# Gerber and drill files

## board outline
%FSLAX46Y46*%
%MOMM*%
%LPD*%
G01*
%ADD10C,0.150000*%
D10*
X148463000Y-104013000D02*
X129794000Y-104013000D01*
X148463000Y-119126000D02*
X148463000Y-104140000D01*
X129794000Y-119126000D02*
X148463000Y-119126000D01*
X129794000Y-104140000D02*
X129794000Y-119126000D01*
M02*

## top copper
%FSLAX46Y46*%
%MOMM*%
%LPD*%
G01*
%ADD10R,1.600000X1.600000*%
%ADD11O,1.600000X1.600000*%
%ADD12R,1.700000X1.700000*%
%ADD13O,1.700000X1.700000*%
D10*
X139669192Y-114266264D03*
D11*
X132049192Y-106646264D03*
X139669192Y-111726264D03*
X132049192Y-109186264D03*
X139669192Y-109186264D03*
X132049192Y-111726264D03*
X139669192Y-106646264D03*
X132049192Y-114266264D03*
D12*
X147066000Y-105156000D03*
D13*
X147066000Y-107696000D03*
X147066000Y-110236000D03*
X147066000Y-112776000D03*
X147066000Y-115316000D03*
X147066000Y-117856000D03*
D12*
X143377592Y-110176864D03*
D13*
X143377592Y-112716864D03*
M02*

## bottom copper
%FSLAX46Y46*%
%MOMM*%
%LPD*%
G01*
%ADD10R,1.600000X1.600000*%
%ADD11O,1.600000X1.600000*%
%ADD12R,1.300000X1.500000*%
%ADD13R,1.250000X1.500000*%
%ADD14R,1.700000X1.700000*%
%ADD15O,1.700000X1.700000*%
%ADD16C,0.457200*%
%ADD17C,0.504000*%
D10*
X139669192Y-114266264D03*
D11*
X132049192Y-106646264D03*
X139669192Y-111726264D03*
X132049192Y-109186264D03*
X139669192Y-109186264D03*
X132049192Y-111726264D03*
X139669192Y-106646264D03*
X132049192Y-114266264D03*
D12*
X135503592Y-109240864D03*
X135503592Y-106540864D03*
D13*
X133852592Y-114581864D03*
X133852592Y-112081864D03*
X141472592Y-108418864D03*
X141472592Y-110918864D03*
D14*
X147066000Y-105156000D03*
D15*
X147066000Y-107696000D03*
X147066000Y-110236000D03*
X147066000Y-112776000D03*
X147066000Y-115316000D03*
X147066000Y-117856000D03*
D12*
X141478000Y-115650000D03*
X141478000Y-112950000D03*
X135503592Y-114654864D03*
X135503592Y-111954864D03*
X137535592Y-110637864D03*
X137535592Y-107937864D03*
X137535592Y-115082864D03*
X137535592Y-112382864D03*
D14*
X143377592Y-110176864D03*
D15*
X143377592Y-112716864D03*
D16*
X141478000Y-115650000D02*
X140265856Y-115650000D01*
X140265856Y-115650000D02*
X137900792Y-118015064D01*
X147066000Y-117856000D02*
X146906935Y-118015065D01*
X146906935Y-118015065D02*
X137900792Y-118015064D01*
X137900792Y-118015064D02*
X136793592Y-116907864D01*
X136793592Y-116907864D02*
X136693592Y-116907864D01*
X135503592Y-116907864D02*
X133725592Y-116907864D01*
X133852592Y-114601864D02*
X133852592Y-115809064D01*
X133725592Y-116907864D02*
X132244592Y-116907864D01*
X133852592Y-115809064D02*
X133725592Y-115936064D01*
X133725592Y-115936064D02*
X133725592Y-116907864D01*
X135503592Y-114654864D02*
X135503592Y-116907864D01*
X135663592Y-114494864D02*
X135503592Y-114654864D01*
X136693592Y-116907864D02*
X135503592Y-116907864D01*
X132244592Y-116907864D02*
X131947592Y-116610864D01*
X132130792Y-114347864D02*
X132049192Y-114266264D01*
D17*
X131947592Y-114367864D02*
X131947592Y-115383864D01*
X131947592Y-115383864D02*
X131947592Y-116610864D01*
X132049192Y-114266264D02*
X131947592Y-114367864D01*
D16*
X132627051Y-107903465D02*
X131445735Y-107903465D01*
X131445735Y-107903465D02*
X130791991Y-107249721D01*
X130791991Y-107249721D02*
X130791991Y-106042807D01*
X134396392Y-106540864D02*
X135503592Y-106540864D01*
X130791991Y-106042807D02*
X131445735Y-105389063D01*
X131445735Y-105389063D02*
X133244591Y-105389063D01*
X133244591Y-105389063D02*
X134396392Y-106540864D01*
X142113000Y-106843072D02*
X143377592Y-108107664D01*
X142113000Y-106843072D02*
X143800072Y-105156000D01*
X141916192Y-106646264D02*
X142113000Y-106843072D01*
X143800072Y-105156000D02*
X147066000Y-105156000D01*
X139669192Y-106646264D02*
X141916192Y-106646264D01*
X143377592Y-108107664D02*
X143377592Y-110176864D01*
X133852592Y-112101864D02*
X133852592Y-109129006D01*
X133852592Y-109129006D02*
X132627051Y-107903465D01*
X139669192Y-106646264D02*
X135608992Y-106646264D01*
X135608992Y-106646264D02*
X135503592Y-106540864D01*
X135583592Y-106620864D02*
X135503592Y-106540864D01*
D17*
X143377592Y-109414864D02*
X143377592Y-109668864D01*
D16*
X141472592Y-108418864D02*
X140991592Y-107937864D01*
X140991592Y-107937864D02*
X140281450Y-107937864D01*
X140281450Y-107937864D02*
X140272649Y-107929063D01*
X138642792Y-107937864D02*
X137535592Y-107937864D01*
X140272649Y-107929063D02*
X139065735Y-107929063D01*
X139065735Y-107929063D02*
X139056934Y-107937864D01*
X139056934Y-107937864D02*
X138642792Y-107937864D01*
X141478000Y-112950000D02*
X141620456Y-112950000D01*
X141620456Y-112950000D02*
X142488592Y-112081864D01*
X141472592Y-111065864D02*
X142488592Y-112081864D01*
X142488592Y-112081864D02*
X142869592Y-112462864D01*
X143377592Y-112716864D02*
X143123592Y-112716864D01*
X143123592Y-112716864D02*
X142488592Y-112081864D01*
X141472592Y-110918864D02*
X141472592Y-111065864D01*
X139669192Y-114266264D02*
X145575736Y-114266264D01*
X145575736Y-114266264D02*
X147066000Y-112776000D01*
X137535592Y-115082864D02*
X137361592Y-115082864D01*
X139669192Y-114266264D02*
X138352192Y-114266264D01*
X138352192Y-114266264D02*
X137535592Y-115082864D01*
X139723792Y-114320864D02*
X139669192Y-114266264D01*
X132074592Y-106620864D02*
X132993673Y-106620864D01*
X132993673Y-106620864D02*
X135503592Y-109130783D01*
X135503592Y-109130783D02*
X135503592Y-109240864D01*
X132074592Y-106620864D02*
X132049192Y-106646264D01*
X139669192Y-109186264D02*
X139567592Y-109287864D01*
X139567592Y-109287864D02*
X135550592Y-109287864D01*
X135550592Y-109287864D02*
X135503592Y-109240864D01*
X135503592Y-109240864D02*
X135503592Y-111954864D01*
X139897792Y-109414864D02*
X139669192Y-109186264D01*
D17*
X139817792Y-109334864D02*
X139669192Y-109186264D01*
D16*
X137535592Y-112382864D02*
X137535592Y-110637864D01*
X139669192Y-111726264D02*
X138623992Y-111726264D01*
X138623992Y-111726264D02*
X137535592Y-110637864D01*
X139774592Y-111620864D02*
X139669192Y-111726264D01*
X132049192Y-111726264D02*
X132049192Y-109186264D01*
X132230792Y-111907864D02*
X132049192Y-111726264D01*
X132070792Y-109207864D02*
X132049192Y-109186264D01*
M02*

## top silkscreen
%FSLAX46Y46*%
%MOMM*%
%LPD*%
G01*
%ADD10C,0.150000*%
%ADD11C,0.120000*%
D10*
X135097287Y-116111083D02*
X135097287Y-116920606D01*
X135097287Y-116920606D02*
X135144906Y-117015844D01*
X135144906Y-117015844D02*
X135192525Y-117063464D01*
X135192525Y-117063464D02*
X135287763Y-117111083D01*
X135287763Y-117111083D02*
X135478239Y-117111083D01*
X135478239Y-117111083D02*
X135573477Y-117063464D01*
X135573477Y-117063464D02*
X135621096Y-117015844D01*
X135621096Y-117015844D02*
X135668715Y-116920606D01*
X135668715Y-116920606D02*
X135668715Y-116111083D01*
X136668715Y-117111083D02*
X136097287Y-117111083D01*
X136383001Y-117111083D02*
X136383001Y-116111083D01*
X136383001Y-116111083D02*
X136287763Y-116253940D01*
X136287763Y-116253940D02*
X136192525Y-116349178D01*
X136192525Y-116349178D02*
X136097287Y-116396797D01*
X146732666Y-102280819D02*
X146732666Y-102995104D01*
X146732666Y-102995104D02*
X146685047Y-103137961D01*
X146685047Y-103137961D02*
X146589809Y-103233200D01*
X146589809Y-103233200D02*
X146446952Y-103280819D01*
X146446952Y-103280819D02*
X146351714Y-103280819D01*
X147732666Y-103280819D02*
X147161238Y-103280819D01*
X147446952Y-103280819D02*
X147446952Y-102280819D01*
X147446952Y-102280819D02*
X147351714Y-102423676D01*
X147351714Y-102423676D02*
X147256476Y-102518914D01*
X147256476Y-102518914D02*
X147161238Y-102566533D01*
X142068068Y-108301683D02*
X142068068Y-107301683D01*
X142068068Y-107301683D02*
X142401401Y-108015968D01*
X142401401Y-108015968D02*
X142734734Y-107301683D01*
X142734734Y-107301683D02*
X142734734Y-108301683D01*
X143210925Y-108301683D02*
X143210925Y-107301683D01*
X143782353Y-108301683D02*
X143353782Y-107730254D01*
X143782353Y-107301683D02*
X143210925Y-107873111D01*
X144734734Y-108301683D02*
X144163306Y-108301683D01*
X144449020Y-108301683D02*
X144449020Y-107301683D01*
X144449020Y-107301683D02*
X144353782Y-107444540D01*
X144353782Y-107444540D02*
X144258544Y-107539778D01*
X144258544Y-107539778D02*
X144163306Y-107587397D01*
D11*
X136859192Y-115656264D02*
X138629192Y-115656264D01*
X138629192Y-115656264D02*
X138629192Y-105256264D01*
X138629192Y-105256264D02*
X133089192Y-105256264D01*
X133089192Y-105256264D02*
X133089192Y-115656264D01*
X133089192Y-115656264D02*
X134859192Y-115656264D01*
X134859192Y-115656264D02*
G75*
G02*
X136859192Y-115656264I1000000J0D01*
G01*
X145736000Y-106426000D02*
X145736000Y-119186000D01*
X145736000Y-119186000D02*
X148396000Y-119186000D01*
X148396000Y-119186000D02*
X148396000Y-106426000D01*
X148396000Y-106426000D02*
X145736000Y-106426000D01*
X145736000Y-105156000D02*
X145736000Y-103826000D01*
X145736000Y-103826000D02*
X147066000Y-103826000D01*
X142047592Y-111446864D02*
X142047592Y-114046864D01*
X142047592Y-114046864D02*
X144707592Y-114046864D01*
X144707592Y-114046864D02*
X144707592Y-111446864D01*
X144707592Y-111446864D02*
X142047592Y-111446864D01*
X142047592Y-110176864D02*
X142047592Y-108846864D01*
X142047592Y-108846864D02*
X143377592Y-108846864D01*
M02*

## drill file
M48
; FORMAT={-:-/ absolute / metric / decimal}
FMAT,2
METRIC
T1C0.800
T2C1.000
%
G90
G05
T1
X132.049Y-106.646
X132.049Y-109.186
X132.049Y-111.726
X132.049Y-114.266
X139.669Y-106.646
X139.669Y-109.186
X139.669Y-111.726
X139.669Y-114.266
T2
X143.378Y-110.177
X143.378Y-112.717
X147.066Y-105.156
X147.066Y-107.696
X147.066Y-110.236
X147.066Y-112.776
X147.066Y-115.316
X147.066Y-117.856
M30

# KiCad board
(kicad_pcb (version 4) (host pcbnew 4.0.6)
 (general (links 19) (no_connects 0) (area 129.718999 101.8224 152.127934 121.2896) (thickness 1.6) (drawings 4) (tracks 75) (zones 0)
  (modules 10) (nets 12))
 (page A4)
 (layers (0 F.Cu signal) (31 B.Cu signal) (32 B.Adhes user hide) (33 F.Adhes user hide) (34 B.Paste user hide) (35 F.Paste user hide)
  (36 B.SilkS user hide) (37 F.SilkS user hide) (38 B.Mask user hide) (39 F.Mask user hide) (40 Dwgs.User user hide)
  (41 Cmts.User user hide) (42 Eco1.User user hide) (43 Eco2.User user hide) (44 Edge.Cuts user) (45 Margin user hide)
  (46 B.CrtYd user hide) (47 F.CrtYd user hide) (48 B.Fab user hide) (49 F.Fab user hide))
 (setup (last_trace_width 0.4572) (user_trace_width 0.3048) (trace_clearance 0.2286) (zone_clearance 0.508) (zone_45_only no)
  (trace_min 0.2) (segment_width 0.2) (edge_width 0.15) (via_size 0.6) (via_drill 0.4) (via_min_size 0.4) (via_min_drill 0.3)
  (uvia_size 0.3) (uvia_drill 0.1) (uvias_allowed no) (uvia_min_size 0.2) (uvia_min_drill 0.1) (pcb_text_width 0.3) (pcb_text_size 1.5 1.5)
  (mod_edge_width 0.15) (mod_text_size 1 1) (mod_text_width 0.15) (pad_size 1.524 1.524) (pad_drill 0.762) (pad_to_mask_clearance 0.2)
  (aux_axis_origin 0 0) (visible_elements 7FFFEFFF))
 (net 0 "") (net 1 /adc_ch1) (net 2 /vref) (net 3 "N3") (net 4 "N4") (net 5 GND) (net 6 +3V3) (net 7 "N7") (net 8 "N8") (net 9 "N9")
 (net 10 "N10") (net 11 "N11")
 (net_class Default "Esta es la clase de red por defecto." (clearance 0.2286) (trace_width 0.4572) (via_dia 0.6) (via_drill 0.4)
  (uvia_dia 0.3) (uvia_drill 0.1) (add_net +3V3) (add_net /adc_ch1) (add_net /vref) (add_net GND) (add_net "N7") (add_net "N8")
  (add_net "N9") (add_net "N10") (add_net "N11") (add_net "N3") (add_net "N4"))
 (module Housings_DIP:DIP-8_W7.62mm (layer F.Cu) (at 139.669192 114.266264 180)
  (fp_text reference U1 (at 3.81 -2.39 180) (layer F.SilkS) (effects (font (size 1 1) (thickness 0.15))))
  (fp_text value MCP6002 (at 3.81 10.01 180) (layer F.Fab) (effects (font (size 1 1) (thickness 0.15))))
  (fp_line (start 2.81 -1.39) (end 1.04 -1.39) (layer F.SilkS) (width 0.12))
  (fp_line (start 1.04 -1.39) (end 1.04 9.01) (layer F.SilkS) (width 0.12))
  (fp_line (start 1.04 9.01) (end 6.58 9.01) (layer F.SilkS) (width 0.12))
  (fp_line (start 6.58 9.01) (end 6.58 -1.39) (layer F.SilkS) (width 0.12))
  (fp_line (start 6.58 -1.39) (end 4.81 -1.39) (layer F.SilkS) (width 0.12))
  (fp_arc (start 3.81 -1.39) (end 2.81 -1.39) (angle -180) (layer F.SilkS) (width 0.12))
  (pad 1 thru_hole rect (at 0 0 180) (size 1.6 1.6) (drill 0.8) (layers *.Cu *.Mask) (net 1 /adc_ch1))
  (pad 5 thru_hole oval (at 7.62 7.62 180) (size 1.6 1.6) (drill 0.8) (layers *.Cu *.Mask) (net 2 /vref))
  (pad 2 thru_hole oval (at 0 2.54 180) (size 1.6 1.6) (drill 0.8) (layers *.Cu *.Mask) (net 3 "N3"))
  (pad 6 thru_hole oval (at 7.62 5.08 180) (size 1.6 1.6) (drill 0.8) (layers *.Cu *.Mask) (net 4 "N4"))
  (pad 3 thru_hole oval (at 0 5.08 180) (size 1.6 1.6) (drill 0.8) (layers *.Cu *.Mask) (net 2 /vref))
  (pad 7 thru_hole oval (at 7.62 2.54 180) (size 1.6 1.6) (drill 0.8) (layers *.Cu *.Mask) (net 4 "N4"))
  (pad 4 thru_hole oval (at 0 7.62 180) (size 1.6 1.6) (drill 0.8) (layers *.Cu *.Mask) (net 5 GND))
  (pad 8 thru_hole oval (at 7.62 0 180) (size 1.6 1.6) (drill 0.8) (layers *.Cu *.Mask) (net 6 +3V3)))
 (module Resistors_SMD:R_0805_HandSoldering (layer B.Cu) (at 135.503592 107.890864 90)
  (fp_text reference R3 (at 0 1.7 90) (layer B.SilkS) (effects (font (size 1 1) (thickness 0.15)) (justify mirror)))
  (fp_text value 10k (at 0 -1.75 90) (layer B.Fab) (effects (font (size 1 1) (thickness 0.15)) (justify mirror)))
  (pad 1 smd rect (at -1.35 0 90) (size 1.5 1.3) (layers B.Cu B.Paste B.Mask) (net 2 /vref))
  (pad 2 smd rect (at 1.35 0 90) (size 1.5 1.3) (layers B.Cu B.Paste B.Mask) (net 5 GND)))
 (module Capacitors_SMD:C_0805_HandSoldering (layer B.Cu) (at 133.852592 113.331864 90)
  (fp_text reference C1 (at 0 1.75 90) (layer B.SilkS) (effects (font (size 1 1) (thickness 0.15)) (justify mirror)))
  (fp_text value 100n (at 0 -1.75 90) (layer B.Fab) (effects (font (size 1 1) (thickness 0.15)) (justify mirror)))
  (pad 1 smd rect (at -1.25 0 90) (size 1.5 1.25) (layers B.Cu B.Paste B.Mask) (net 6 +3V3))
  (pad 2 smd rect (at 1.25 0 90) (size 1.5 1.25) (layers B.Cu B.Paste B.Mask) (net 5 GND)))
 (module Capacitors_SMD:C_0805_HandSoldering (layer B.Cu) (at 141.472592 109.668864 270)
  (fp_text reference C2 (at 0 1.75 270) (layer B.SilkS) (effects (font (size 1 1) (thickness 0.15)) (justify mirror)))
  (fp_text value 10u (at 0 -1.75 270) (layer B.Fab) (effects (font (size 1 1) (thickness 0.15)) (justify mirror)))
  (pad 1 smd rect (at -1.25 0 270) (size 1.5 1.25) (layers B.Cu B.Paste B.Mask) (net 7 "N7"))
  (pad 2 smd rect (at 1.25 0 270) (size 1.5 1.25) (layers B.Cu B.Paste B.Mask) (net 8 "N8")))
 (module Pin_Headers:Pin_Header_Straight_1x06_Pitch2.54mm (layer F.Cu) (at 147.066 105.156)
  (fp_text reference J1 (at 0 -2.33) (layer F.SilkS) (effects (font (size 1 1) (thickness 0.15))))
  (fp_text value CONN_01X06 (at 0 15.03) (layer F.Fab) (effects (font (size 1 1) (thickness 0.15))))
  (fp_line (start -1.33 1.27) (end -1.33 14.03) (layer F.SilkS) (width 0.12))
  (fp_line (start -1.33 14.03) (end 1.33 14.03) (layer F.SilkS) (width 0.12))
  (fp_line (start 1.33 14.03) (end 1.33 1.27) (layer F.SilkS) (width 0.12))
  (fp_line (start 1.33 1.27) (end -1.33 1.27) (layer F.SilkS) (width 0.12))
  (fp_line (start -1.33 0) (end -1.33 -1.33) (layer F.SilkS) (width 0.12))
  (fp_line (start -1.33 -1.33) (end 0 -1.33) (layer F.SilkS) (width 0.12))
  (pad 1 thru_hole rect (at 0 0) (size 1.7 1.7) (drill 1) (layers *.Cu *.Mask) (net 5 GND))
  (pad 2 thru_hole oval (at 0 2.54) (size 1.7 1.7) (drill 1) (layers *.Cu *.Mask) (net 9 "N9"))
  (pad 3 thru_hole oval (at 0 5.08) (size 1.7 1.7) (drill 1) (layers *.Cu *.Mask) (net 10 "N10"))
  (pad 4 thru_hole oval (at 0 7.62) (size 1.7 1.7) (drill 1) (layers *.Cu *.Mask) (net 1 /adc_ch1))
  (pad 5 thru_hole oval (at 0 10.16) (size 1.7 1.7) (drill 1) (layers *.Cu *.Mask) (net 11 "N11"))
  (pad 6 thru_hole oval (at 0 12.7) (size 1.7 1.7) (drill 1) (layers *.Cu *.Mask) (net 6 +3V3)))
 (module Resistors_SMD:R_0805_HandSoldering (layer B.Cu) (at 141.478 114.3 90)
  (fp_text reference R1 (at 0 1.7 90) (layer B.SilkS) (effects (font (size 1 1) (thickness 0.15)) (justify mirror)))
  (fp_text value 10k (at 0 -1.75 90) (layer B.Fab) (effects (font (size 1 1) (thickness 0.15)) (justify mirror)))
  (pad 1 smd rect (at -1.35 0 90) (size 1.5 1.3) (layers B.Cu B.Paste B.Mask) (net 6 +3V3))
  (pad 2 smd rect (at 1.35 0 90) (size 1.5 1.3) (layers B.Cu B.Paste B.Mask) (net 8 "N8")))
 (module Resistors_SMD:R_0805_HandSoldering (layer B.Cu) (at 135.503592 113.304864 90)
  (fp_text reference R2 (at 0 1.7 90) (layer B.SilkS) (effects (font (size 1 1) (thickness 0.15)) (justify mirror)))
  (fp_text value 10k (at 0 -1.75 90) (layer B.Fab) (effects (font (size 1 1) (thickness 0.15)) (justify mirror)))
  (pad 1 smd rect (at -1.35 0 90) (size 1.5 1.3) (layers B.Cu B.Paste B.Mask) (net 6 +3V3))
  (pad 2 smd rect (at 1.35 0 90) (size 1.5 1.3) (layers B.Cu B.Paste B.Mask) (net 2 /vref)))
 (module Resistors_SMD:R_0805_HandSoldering (layer B.Cu) (at 137.535592 109.287864 90)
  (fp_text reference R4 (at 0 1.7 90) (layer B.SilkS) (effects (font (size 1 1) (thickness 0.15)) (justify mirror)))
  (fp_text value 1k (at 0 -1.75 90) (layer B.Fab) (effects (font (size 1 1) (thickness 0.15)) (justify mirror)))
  (pad 1 smd rect (at -1.35 0 90) (size 1.5 1.3) (layers B.Cu B.Paste B.Mask) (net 3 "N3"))
  (pad 2 smd rect (at 1.35 0 90) (size 1.5 1.3) (layers B.Cu B.Paste B.Mask) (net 7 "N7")))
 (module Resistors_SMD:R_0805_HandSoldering (layer B.Cu) (at 137.535592 113.732864 90)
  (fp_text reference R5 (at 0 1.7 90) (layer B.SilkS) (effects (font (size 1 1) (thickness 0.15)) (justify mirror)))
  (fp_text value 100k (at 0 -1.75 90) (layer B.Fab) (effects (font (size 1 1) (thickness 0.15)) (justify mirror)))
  (pad 1 smd rect (at -1.35 0 90) (size 1.5 1.3) (layers B.Cu B.Paste B.Mask) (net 1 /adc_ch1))
  (pad 2 smd rect (at 1.35 0 90) (size 1.5 1.3) (layers B.Cu B.Paste B.Mask) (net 3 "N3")))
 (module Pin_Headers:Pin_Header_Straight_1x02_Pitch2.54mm (layer F.Cu) (at 143.377592 110.176864)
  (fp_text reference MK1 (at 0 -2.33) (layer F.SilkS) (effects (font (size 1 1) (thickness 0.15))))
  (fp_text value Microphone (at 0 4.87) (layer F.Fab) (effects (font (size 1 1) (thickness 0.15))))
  (fp_line (start -1.33 1.27) (end -1.33 3.87) (layer F.SilkS) (width 0.12))
  (fp_line (start -1.33 3.87) (end 1.33 3.87) (layer F.SilkS) (width 0.12))
  (fp_line (start 1.33 3.87) (end 1.33 1.27) (layer F.SilkS) (width 0.12))
  (fp_line (start 1.33 1.27) (end -1.33 1.27) (layer F.SilkS) (width 0.12))
  (fp_line (start -1.33 0) (end -1.33 -1.33) (layer F.SilkS) (width 0.12))
  (fp_line (start -1.33 -1.33) (end 0 -1.33) (layer F.SilkS) (width 0.12))
  (pad 1 thru_hole rect (at 0 0) (size 1.7 1.7) (drill 1) (layers *.Cu *.Mask) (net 5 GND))
  (pad 2 thru_hole oval (at 0 2.54) (size 1.7 1.7) (drill 1) (layers *.Cu *.Mask) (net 8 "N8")))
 (gr_line (start 148.463 104.013) (end 129.794 104.013) (layer Edge.Cuts) (width 0.15))
 (gr_line (start 148.463 119.126) (end 148.463 104.14) (layer Edge.Cuts) (width 0.15))
 (gr_line (start 129.794 119.126) (end 148.463 119.126) (layer Edge.Cuts) (width 0.15))
 (gr_line (start 129.794 104.14) (end 129.794 119.126) (layer Edge.Cuts) (width 0.15))
 (segment (start 141.478 115.65) (end 140.265856 115.65) (width 0.4572) (layer B.Cu) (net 6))
 (segment (start 140.265856 115.65) (end 137.900792 118.015064) (width 0.4572) (layer B.Cu) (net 6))
 (segment (start 147.066 117.856) (end 146.906935 118.015065) (width 0.4572) (layer B.Cu) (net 6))
 (segment (start 146.906935 118.015065) (end 137.900792 118.015064) (width 0.4572) (layer B.Cu) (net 6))
 (segment (start 137.900792 118.015064) (end 136.793592 116.907864) (width 0.4572) (layer B.Cu) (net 6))
 (segment (start 136.793592 116.907864) (end 136.693592 116.907864) (width 0.4572) (layer B.Cu) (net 6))
 (segment (start 135.503592 116.907864) (end 133.725592 116.907864) (width 0.4572) (layer B.Cu) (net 6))
 (segment (start 133.852592 114.601864) (end 133.852592 115.809064) (width 0.4572) (layer B.Cu) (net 6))
 (segment (start 133.725592 116.907864) (end 132.244592 116.907864) (width 0.4572) (layer B.Cu) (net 6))
 (segment (start 133.852592 115.809064) (end 133.725592 115.936064) (width 0.4572) (layer B.Cu) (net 6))
 (segment (start 133.725592 115.936064) (end 133.725592 116.907864) (width 0.4572) (layer B.Cu) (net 6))
 (segment (start 135.503592 114.654864) (end 135.503592 116.907864) (width 0.4572) (layer B.Cu) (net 6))
 (segment (start 135.663592 114.494864) (end 135.503592 114.654864) (width 0.4572) (layer B.Cu) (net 6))
 (segment (start 136.693592 116.907864) (end 135.503592 116.907864) (width 0.4572) (layer B.Cu) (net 6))
 (segment (start 132.244592 116.907864) (end 131.947592 116.610864) (width 0.4572) (layer B.Cu) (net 6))
 (segment (start 132.130792 114.347864) (end 132.049192 114.266264) (width 0.4572) (layer B.Cu) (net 6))
 (segment (start 131.947592 114.367864) (end 131.947592 115.383864) (width 0.504) (layer B.Cu) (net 6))
 (segment (start 131.947592 115.383864) (end 131.947592 116.610864) (width 0.504) (layer B.Cu) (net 6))
 (segment (start 132.049192 114.266264) (end 131.947592 114.367864) (width 0.504) (layer B.Cu) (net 6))
 (segment (start 132.627051 107.903465) (end 131.445735 107.903465) (width 0.4572) (layer B.Cu) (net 5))
 (segment (start 131.445735 107.903465) (end 130.791991 107.249721) (width 0.4572) (layer B.Cu) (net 5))
 (segment (start 130.791991 107.249721) (end 130.791991 106.042807) (width 0.4572) (layer B.Cu) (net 5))
 (segment (start 134.396392 106.540864) (end 135.503592 106.540864) (width 0.4572) (layer B.Cu) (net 5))
 (segment (start 130.791991 106.042807) (end 131.445735 105.389063) (width 0.4572) (layer B.Cu) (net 5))
 (segment (start 131.445735 105.389063) (end 133.244591 105.389063) (width 0.4572) (layer B.Cu) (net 5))
 (segment (start 133.244591 105.389063) (end 134.396392 106.540864) (width 0.4572) (layer B.Cu) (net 5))
 (segment (start 142.113 106.843072) (end 143.377592 108.107664) (width 0.4572) (layer B.Cu) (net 5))
 (segment (start 142.113 106.843072) (end 143.800072 105.156) (width 0.4572) (layer B.Cu) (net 5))
 (segment (start 141.916192 106.646264) (end 142.113 106.843072) (width 0.4572) (layer B.Cu) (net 5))
 (segment (start 143.800072 105.156) (end 147.066 105.156) (width 0.4572) (layer B.Cu) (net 5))
 (segment (start 139.669192 106.646264) (end 141.916192 106.646264) (width 0.4572) (layer B.Cu) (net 5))
 (segment (start 143.377592 108.107664) (end 143.377592 110.176864) (width 0.4572) (layer B.Cu) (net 5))
 (segment (start 133.852592 112.101864) (end 133.852592 109.129006) (width 0.4572) (layer B.Cu) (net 5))
 (segment (start 133.852592 109.129006) (end 132.627051 107.903465) (width 0.4572) (layer B.Cu) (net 5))
 (segment (start 139.669192 106.646264) (end 135.608992 106.646264) (width 0.4572) (layer B.Cu) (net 5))
 (segment (start 135.608992 106.646264) (end 135.503592 106.540864) (width 0.4572) (layer B.Cu) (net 5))
 (segment (start 135.583592 106.620864) (end 135.503592 106.540864) (width 0.4572) (layer B.Cu) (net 5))
 (segment (start 143.377592 109.414864) (end 143.377592 109.668864) (width 0.504) (layer B.Cu) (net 5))
 (segment (start 141.472592 108.418864) (end 140.991592 107.937864) (width 0.4572) (layer B.Cu) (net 7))
 (segment (start 140.991592 107.937864) (end 140.28145 107.937864) (width 0.4572) (layer B.Cu) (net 7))
 (segment (start 140.28145 107.937864) (end 140.272649 107.929063) (width 0.4572) (layer B.Cu) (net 7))
 (segment (start 138.642792 107.937864) (end 137.535592 107.937864) (width 0.4572) (layer B.Cu) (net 7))
 (segment (start 140.272649 107.929063) (end 139.065735 107.929063) (width 0.4572) (layer B.Cu) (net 7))
 (segment (start 139.065735 107.929063) (end 139.056934 107.937864) (width 0.4572) (layer B.Cu) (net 7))
 (segment (start 139.056934 107.937864) (end 138.642792 107.937864) (width 0.4572) (layer B.Cu) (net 7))
 (segment (start 141.478 112.95) (end 141.620456 112.95) (width 0.4572) (layer B.Cu) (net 8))
 (segment (start 141.620456 112.95) (end 142.488592 112.081864) (width 0.4572) (layer B.Cu) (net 8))
 (segment (start 141.472592 111.065864) (end 142.488592 112.081864) (width 0.4572) (layer B.Cu) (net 8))
 (segment (start 142.488592 112.081864) (end 142.869592 112.462864) (width 0.4572) (layer B.Cu) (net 8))
 (segment (start 143.377592 112.716864) (end 143.123592 112.716864) (width 0.4572) (layer B.Cu) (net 8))
 (segment (start 143.123592 112.716864) (end 142.488592 112.081864) (width 0.4572) (layer B.Cu) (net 8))
 (segment (start 141.472592 110.918864) (end 141.472592 111.065864) (width 0.4572) (layer B.Cu) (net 8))
 (segment (start 139.669192 114.266264) (end 145.575736 114.266264) (width 0.4572) (layer B.Cu) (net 1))
 (segment (start 145.575736 114.266264) (end 147.066 112.776) (width 0.4572) (layer B.Cu) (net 1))
 (segment (start 137.535592 115.082864) (end 137.361592 115.082864) (width 0.4572) (layer B.Cu) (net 1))
 (segment (start 139.669192 114.266264) (end 138.352192 114.266264) (width 0.4572) (layer B.Cu) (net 1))
 (segment (start 138.352192 114.266264) (end 137.535592 115.082864) (width 0.4572) (layer B.Cu) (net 1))
 (segment (start 139.723792 114.320864) (end 139.669192 114.266264) (width 0.4572) (layer B.Cu) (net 1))
 (segment (start 132.074592 106.620864) (end 132.993673 106.620864) (width 0.4572) (layer B.Cu) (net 2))
 (segment (start 132.993673 106.620864) (end 135.503592 109.130783) (width 0.4572) (layer B.Cu) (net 2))
 (segment (start 135.503592 109.130783) (end 135.503592 109.240864) (width 0.4572) (layer B.Cu) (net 2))
 (segment (start 132.074592 106.620864) (end 132.049192 106.646264) (width 0.4572) (layer B.Cu) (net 2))
 (segment (start 139.669192 109.186264) (end 139.567592 109.287864) (width 0.4572) (layer B.Cu) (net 2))
 (segment (start 139.567592 109.287864) (end 135.550592 109.287864) (width 0.4572) (layer B.Cu) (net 2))
 (segment (start 135.550592 109.287864) (end 135.503592 109.240864) (width 0.4572) (layer B.Cu) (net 2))
 (segment (start 135.503592 109.240864) (end 135.503592 111.954864) (width 0.4572) (layer B.Cu) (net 2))
 (segment (start 139.897792 109.414864) (end 139.669192 109.186264) (width 0.4572) (layer B.Cu) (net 2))
 (segment (start 139.817792 109.334864) (end 139.669192 109.186264) (width 0.504) (layer B.Cu) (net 2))
 (segment (start 137.535592 112.382864) (end 137.535592 110.637864) (width 0.4572) (layer B.Cu) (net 3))
 (segment (start 139.669192 111.726264) (end 138.623992 111.726264) (width 0.4572) (layer B.Cu) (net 3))
 (segment (start 138.623992 111.726264) (end 137.535592 110.637864) (width 0.4572) (layer B.Cu) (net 3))
 (segment (start 139.774592 111.620864) (end 139.669192 111.726264) (width 0.4572) (layer B.Cu) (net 3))
 (segment (start 132.049192 111.726264) (end 132.049192 109.186264) (width 0.4572) (layer B.Cu) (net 4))
 (segment (start 132.230792 111.907864) (end 132.049192 111.726264) (width 0.4572) (layer B.Cu) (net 4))
 (segment (start 132.070792 109.207864) (end 132.049192 109.186264) (width 0.4572) (layer B.Cu) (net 4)))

